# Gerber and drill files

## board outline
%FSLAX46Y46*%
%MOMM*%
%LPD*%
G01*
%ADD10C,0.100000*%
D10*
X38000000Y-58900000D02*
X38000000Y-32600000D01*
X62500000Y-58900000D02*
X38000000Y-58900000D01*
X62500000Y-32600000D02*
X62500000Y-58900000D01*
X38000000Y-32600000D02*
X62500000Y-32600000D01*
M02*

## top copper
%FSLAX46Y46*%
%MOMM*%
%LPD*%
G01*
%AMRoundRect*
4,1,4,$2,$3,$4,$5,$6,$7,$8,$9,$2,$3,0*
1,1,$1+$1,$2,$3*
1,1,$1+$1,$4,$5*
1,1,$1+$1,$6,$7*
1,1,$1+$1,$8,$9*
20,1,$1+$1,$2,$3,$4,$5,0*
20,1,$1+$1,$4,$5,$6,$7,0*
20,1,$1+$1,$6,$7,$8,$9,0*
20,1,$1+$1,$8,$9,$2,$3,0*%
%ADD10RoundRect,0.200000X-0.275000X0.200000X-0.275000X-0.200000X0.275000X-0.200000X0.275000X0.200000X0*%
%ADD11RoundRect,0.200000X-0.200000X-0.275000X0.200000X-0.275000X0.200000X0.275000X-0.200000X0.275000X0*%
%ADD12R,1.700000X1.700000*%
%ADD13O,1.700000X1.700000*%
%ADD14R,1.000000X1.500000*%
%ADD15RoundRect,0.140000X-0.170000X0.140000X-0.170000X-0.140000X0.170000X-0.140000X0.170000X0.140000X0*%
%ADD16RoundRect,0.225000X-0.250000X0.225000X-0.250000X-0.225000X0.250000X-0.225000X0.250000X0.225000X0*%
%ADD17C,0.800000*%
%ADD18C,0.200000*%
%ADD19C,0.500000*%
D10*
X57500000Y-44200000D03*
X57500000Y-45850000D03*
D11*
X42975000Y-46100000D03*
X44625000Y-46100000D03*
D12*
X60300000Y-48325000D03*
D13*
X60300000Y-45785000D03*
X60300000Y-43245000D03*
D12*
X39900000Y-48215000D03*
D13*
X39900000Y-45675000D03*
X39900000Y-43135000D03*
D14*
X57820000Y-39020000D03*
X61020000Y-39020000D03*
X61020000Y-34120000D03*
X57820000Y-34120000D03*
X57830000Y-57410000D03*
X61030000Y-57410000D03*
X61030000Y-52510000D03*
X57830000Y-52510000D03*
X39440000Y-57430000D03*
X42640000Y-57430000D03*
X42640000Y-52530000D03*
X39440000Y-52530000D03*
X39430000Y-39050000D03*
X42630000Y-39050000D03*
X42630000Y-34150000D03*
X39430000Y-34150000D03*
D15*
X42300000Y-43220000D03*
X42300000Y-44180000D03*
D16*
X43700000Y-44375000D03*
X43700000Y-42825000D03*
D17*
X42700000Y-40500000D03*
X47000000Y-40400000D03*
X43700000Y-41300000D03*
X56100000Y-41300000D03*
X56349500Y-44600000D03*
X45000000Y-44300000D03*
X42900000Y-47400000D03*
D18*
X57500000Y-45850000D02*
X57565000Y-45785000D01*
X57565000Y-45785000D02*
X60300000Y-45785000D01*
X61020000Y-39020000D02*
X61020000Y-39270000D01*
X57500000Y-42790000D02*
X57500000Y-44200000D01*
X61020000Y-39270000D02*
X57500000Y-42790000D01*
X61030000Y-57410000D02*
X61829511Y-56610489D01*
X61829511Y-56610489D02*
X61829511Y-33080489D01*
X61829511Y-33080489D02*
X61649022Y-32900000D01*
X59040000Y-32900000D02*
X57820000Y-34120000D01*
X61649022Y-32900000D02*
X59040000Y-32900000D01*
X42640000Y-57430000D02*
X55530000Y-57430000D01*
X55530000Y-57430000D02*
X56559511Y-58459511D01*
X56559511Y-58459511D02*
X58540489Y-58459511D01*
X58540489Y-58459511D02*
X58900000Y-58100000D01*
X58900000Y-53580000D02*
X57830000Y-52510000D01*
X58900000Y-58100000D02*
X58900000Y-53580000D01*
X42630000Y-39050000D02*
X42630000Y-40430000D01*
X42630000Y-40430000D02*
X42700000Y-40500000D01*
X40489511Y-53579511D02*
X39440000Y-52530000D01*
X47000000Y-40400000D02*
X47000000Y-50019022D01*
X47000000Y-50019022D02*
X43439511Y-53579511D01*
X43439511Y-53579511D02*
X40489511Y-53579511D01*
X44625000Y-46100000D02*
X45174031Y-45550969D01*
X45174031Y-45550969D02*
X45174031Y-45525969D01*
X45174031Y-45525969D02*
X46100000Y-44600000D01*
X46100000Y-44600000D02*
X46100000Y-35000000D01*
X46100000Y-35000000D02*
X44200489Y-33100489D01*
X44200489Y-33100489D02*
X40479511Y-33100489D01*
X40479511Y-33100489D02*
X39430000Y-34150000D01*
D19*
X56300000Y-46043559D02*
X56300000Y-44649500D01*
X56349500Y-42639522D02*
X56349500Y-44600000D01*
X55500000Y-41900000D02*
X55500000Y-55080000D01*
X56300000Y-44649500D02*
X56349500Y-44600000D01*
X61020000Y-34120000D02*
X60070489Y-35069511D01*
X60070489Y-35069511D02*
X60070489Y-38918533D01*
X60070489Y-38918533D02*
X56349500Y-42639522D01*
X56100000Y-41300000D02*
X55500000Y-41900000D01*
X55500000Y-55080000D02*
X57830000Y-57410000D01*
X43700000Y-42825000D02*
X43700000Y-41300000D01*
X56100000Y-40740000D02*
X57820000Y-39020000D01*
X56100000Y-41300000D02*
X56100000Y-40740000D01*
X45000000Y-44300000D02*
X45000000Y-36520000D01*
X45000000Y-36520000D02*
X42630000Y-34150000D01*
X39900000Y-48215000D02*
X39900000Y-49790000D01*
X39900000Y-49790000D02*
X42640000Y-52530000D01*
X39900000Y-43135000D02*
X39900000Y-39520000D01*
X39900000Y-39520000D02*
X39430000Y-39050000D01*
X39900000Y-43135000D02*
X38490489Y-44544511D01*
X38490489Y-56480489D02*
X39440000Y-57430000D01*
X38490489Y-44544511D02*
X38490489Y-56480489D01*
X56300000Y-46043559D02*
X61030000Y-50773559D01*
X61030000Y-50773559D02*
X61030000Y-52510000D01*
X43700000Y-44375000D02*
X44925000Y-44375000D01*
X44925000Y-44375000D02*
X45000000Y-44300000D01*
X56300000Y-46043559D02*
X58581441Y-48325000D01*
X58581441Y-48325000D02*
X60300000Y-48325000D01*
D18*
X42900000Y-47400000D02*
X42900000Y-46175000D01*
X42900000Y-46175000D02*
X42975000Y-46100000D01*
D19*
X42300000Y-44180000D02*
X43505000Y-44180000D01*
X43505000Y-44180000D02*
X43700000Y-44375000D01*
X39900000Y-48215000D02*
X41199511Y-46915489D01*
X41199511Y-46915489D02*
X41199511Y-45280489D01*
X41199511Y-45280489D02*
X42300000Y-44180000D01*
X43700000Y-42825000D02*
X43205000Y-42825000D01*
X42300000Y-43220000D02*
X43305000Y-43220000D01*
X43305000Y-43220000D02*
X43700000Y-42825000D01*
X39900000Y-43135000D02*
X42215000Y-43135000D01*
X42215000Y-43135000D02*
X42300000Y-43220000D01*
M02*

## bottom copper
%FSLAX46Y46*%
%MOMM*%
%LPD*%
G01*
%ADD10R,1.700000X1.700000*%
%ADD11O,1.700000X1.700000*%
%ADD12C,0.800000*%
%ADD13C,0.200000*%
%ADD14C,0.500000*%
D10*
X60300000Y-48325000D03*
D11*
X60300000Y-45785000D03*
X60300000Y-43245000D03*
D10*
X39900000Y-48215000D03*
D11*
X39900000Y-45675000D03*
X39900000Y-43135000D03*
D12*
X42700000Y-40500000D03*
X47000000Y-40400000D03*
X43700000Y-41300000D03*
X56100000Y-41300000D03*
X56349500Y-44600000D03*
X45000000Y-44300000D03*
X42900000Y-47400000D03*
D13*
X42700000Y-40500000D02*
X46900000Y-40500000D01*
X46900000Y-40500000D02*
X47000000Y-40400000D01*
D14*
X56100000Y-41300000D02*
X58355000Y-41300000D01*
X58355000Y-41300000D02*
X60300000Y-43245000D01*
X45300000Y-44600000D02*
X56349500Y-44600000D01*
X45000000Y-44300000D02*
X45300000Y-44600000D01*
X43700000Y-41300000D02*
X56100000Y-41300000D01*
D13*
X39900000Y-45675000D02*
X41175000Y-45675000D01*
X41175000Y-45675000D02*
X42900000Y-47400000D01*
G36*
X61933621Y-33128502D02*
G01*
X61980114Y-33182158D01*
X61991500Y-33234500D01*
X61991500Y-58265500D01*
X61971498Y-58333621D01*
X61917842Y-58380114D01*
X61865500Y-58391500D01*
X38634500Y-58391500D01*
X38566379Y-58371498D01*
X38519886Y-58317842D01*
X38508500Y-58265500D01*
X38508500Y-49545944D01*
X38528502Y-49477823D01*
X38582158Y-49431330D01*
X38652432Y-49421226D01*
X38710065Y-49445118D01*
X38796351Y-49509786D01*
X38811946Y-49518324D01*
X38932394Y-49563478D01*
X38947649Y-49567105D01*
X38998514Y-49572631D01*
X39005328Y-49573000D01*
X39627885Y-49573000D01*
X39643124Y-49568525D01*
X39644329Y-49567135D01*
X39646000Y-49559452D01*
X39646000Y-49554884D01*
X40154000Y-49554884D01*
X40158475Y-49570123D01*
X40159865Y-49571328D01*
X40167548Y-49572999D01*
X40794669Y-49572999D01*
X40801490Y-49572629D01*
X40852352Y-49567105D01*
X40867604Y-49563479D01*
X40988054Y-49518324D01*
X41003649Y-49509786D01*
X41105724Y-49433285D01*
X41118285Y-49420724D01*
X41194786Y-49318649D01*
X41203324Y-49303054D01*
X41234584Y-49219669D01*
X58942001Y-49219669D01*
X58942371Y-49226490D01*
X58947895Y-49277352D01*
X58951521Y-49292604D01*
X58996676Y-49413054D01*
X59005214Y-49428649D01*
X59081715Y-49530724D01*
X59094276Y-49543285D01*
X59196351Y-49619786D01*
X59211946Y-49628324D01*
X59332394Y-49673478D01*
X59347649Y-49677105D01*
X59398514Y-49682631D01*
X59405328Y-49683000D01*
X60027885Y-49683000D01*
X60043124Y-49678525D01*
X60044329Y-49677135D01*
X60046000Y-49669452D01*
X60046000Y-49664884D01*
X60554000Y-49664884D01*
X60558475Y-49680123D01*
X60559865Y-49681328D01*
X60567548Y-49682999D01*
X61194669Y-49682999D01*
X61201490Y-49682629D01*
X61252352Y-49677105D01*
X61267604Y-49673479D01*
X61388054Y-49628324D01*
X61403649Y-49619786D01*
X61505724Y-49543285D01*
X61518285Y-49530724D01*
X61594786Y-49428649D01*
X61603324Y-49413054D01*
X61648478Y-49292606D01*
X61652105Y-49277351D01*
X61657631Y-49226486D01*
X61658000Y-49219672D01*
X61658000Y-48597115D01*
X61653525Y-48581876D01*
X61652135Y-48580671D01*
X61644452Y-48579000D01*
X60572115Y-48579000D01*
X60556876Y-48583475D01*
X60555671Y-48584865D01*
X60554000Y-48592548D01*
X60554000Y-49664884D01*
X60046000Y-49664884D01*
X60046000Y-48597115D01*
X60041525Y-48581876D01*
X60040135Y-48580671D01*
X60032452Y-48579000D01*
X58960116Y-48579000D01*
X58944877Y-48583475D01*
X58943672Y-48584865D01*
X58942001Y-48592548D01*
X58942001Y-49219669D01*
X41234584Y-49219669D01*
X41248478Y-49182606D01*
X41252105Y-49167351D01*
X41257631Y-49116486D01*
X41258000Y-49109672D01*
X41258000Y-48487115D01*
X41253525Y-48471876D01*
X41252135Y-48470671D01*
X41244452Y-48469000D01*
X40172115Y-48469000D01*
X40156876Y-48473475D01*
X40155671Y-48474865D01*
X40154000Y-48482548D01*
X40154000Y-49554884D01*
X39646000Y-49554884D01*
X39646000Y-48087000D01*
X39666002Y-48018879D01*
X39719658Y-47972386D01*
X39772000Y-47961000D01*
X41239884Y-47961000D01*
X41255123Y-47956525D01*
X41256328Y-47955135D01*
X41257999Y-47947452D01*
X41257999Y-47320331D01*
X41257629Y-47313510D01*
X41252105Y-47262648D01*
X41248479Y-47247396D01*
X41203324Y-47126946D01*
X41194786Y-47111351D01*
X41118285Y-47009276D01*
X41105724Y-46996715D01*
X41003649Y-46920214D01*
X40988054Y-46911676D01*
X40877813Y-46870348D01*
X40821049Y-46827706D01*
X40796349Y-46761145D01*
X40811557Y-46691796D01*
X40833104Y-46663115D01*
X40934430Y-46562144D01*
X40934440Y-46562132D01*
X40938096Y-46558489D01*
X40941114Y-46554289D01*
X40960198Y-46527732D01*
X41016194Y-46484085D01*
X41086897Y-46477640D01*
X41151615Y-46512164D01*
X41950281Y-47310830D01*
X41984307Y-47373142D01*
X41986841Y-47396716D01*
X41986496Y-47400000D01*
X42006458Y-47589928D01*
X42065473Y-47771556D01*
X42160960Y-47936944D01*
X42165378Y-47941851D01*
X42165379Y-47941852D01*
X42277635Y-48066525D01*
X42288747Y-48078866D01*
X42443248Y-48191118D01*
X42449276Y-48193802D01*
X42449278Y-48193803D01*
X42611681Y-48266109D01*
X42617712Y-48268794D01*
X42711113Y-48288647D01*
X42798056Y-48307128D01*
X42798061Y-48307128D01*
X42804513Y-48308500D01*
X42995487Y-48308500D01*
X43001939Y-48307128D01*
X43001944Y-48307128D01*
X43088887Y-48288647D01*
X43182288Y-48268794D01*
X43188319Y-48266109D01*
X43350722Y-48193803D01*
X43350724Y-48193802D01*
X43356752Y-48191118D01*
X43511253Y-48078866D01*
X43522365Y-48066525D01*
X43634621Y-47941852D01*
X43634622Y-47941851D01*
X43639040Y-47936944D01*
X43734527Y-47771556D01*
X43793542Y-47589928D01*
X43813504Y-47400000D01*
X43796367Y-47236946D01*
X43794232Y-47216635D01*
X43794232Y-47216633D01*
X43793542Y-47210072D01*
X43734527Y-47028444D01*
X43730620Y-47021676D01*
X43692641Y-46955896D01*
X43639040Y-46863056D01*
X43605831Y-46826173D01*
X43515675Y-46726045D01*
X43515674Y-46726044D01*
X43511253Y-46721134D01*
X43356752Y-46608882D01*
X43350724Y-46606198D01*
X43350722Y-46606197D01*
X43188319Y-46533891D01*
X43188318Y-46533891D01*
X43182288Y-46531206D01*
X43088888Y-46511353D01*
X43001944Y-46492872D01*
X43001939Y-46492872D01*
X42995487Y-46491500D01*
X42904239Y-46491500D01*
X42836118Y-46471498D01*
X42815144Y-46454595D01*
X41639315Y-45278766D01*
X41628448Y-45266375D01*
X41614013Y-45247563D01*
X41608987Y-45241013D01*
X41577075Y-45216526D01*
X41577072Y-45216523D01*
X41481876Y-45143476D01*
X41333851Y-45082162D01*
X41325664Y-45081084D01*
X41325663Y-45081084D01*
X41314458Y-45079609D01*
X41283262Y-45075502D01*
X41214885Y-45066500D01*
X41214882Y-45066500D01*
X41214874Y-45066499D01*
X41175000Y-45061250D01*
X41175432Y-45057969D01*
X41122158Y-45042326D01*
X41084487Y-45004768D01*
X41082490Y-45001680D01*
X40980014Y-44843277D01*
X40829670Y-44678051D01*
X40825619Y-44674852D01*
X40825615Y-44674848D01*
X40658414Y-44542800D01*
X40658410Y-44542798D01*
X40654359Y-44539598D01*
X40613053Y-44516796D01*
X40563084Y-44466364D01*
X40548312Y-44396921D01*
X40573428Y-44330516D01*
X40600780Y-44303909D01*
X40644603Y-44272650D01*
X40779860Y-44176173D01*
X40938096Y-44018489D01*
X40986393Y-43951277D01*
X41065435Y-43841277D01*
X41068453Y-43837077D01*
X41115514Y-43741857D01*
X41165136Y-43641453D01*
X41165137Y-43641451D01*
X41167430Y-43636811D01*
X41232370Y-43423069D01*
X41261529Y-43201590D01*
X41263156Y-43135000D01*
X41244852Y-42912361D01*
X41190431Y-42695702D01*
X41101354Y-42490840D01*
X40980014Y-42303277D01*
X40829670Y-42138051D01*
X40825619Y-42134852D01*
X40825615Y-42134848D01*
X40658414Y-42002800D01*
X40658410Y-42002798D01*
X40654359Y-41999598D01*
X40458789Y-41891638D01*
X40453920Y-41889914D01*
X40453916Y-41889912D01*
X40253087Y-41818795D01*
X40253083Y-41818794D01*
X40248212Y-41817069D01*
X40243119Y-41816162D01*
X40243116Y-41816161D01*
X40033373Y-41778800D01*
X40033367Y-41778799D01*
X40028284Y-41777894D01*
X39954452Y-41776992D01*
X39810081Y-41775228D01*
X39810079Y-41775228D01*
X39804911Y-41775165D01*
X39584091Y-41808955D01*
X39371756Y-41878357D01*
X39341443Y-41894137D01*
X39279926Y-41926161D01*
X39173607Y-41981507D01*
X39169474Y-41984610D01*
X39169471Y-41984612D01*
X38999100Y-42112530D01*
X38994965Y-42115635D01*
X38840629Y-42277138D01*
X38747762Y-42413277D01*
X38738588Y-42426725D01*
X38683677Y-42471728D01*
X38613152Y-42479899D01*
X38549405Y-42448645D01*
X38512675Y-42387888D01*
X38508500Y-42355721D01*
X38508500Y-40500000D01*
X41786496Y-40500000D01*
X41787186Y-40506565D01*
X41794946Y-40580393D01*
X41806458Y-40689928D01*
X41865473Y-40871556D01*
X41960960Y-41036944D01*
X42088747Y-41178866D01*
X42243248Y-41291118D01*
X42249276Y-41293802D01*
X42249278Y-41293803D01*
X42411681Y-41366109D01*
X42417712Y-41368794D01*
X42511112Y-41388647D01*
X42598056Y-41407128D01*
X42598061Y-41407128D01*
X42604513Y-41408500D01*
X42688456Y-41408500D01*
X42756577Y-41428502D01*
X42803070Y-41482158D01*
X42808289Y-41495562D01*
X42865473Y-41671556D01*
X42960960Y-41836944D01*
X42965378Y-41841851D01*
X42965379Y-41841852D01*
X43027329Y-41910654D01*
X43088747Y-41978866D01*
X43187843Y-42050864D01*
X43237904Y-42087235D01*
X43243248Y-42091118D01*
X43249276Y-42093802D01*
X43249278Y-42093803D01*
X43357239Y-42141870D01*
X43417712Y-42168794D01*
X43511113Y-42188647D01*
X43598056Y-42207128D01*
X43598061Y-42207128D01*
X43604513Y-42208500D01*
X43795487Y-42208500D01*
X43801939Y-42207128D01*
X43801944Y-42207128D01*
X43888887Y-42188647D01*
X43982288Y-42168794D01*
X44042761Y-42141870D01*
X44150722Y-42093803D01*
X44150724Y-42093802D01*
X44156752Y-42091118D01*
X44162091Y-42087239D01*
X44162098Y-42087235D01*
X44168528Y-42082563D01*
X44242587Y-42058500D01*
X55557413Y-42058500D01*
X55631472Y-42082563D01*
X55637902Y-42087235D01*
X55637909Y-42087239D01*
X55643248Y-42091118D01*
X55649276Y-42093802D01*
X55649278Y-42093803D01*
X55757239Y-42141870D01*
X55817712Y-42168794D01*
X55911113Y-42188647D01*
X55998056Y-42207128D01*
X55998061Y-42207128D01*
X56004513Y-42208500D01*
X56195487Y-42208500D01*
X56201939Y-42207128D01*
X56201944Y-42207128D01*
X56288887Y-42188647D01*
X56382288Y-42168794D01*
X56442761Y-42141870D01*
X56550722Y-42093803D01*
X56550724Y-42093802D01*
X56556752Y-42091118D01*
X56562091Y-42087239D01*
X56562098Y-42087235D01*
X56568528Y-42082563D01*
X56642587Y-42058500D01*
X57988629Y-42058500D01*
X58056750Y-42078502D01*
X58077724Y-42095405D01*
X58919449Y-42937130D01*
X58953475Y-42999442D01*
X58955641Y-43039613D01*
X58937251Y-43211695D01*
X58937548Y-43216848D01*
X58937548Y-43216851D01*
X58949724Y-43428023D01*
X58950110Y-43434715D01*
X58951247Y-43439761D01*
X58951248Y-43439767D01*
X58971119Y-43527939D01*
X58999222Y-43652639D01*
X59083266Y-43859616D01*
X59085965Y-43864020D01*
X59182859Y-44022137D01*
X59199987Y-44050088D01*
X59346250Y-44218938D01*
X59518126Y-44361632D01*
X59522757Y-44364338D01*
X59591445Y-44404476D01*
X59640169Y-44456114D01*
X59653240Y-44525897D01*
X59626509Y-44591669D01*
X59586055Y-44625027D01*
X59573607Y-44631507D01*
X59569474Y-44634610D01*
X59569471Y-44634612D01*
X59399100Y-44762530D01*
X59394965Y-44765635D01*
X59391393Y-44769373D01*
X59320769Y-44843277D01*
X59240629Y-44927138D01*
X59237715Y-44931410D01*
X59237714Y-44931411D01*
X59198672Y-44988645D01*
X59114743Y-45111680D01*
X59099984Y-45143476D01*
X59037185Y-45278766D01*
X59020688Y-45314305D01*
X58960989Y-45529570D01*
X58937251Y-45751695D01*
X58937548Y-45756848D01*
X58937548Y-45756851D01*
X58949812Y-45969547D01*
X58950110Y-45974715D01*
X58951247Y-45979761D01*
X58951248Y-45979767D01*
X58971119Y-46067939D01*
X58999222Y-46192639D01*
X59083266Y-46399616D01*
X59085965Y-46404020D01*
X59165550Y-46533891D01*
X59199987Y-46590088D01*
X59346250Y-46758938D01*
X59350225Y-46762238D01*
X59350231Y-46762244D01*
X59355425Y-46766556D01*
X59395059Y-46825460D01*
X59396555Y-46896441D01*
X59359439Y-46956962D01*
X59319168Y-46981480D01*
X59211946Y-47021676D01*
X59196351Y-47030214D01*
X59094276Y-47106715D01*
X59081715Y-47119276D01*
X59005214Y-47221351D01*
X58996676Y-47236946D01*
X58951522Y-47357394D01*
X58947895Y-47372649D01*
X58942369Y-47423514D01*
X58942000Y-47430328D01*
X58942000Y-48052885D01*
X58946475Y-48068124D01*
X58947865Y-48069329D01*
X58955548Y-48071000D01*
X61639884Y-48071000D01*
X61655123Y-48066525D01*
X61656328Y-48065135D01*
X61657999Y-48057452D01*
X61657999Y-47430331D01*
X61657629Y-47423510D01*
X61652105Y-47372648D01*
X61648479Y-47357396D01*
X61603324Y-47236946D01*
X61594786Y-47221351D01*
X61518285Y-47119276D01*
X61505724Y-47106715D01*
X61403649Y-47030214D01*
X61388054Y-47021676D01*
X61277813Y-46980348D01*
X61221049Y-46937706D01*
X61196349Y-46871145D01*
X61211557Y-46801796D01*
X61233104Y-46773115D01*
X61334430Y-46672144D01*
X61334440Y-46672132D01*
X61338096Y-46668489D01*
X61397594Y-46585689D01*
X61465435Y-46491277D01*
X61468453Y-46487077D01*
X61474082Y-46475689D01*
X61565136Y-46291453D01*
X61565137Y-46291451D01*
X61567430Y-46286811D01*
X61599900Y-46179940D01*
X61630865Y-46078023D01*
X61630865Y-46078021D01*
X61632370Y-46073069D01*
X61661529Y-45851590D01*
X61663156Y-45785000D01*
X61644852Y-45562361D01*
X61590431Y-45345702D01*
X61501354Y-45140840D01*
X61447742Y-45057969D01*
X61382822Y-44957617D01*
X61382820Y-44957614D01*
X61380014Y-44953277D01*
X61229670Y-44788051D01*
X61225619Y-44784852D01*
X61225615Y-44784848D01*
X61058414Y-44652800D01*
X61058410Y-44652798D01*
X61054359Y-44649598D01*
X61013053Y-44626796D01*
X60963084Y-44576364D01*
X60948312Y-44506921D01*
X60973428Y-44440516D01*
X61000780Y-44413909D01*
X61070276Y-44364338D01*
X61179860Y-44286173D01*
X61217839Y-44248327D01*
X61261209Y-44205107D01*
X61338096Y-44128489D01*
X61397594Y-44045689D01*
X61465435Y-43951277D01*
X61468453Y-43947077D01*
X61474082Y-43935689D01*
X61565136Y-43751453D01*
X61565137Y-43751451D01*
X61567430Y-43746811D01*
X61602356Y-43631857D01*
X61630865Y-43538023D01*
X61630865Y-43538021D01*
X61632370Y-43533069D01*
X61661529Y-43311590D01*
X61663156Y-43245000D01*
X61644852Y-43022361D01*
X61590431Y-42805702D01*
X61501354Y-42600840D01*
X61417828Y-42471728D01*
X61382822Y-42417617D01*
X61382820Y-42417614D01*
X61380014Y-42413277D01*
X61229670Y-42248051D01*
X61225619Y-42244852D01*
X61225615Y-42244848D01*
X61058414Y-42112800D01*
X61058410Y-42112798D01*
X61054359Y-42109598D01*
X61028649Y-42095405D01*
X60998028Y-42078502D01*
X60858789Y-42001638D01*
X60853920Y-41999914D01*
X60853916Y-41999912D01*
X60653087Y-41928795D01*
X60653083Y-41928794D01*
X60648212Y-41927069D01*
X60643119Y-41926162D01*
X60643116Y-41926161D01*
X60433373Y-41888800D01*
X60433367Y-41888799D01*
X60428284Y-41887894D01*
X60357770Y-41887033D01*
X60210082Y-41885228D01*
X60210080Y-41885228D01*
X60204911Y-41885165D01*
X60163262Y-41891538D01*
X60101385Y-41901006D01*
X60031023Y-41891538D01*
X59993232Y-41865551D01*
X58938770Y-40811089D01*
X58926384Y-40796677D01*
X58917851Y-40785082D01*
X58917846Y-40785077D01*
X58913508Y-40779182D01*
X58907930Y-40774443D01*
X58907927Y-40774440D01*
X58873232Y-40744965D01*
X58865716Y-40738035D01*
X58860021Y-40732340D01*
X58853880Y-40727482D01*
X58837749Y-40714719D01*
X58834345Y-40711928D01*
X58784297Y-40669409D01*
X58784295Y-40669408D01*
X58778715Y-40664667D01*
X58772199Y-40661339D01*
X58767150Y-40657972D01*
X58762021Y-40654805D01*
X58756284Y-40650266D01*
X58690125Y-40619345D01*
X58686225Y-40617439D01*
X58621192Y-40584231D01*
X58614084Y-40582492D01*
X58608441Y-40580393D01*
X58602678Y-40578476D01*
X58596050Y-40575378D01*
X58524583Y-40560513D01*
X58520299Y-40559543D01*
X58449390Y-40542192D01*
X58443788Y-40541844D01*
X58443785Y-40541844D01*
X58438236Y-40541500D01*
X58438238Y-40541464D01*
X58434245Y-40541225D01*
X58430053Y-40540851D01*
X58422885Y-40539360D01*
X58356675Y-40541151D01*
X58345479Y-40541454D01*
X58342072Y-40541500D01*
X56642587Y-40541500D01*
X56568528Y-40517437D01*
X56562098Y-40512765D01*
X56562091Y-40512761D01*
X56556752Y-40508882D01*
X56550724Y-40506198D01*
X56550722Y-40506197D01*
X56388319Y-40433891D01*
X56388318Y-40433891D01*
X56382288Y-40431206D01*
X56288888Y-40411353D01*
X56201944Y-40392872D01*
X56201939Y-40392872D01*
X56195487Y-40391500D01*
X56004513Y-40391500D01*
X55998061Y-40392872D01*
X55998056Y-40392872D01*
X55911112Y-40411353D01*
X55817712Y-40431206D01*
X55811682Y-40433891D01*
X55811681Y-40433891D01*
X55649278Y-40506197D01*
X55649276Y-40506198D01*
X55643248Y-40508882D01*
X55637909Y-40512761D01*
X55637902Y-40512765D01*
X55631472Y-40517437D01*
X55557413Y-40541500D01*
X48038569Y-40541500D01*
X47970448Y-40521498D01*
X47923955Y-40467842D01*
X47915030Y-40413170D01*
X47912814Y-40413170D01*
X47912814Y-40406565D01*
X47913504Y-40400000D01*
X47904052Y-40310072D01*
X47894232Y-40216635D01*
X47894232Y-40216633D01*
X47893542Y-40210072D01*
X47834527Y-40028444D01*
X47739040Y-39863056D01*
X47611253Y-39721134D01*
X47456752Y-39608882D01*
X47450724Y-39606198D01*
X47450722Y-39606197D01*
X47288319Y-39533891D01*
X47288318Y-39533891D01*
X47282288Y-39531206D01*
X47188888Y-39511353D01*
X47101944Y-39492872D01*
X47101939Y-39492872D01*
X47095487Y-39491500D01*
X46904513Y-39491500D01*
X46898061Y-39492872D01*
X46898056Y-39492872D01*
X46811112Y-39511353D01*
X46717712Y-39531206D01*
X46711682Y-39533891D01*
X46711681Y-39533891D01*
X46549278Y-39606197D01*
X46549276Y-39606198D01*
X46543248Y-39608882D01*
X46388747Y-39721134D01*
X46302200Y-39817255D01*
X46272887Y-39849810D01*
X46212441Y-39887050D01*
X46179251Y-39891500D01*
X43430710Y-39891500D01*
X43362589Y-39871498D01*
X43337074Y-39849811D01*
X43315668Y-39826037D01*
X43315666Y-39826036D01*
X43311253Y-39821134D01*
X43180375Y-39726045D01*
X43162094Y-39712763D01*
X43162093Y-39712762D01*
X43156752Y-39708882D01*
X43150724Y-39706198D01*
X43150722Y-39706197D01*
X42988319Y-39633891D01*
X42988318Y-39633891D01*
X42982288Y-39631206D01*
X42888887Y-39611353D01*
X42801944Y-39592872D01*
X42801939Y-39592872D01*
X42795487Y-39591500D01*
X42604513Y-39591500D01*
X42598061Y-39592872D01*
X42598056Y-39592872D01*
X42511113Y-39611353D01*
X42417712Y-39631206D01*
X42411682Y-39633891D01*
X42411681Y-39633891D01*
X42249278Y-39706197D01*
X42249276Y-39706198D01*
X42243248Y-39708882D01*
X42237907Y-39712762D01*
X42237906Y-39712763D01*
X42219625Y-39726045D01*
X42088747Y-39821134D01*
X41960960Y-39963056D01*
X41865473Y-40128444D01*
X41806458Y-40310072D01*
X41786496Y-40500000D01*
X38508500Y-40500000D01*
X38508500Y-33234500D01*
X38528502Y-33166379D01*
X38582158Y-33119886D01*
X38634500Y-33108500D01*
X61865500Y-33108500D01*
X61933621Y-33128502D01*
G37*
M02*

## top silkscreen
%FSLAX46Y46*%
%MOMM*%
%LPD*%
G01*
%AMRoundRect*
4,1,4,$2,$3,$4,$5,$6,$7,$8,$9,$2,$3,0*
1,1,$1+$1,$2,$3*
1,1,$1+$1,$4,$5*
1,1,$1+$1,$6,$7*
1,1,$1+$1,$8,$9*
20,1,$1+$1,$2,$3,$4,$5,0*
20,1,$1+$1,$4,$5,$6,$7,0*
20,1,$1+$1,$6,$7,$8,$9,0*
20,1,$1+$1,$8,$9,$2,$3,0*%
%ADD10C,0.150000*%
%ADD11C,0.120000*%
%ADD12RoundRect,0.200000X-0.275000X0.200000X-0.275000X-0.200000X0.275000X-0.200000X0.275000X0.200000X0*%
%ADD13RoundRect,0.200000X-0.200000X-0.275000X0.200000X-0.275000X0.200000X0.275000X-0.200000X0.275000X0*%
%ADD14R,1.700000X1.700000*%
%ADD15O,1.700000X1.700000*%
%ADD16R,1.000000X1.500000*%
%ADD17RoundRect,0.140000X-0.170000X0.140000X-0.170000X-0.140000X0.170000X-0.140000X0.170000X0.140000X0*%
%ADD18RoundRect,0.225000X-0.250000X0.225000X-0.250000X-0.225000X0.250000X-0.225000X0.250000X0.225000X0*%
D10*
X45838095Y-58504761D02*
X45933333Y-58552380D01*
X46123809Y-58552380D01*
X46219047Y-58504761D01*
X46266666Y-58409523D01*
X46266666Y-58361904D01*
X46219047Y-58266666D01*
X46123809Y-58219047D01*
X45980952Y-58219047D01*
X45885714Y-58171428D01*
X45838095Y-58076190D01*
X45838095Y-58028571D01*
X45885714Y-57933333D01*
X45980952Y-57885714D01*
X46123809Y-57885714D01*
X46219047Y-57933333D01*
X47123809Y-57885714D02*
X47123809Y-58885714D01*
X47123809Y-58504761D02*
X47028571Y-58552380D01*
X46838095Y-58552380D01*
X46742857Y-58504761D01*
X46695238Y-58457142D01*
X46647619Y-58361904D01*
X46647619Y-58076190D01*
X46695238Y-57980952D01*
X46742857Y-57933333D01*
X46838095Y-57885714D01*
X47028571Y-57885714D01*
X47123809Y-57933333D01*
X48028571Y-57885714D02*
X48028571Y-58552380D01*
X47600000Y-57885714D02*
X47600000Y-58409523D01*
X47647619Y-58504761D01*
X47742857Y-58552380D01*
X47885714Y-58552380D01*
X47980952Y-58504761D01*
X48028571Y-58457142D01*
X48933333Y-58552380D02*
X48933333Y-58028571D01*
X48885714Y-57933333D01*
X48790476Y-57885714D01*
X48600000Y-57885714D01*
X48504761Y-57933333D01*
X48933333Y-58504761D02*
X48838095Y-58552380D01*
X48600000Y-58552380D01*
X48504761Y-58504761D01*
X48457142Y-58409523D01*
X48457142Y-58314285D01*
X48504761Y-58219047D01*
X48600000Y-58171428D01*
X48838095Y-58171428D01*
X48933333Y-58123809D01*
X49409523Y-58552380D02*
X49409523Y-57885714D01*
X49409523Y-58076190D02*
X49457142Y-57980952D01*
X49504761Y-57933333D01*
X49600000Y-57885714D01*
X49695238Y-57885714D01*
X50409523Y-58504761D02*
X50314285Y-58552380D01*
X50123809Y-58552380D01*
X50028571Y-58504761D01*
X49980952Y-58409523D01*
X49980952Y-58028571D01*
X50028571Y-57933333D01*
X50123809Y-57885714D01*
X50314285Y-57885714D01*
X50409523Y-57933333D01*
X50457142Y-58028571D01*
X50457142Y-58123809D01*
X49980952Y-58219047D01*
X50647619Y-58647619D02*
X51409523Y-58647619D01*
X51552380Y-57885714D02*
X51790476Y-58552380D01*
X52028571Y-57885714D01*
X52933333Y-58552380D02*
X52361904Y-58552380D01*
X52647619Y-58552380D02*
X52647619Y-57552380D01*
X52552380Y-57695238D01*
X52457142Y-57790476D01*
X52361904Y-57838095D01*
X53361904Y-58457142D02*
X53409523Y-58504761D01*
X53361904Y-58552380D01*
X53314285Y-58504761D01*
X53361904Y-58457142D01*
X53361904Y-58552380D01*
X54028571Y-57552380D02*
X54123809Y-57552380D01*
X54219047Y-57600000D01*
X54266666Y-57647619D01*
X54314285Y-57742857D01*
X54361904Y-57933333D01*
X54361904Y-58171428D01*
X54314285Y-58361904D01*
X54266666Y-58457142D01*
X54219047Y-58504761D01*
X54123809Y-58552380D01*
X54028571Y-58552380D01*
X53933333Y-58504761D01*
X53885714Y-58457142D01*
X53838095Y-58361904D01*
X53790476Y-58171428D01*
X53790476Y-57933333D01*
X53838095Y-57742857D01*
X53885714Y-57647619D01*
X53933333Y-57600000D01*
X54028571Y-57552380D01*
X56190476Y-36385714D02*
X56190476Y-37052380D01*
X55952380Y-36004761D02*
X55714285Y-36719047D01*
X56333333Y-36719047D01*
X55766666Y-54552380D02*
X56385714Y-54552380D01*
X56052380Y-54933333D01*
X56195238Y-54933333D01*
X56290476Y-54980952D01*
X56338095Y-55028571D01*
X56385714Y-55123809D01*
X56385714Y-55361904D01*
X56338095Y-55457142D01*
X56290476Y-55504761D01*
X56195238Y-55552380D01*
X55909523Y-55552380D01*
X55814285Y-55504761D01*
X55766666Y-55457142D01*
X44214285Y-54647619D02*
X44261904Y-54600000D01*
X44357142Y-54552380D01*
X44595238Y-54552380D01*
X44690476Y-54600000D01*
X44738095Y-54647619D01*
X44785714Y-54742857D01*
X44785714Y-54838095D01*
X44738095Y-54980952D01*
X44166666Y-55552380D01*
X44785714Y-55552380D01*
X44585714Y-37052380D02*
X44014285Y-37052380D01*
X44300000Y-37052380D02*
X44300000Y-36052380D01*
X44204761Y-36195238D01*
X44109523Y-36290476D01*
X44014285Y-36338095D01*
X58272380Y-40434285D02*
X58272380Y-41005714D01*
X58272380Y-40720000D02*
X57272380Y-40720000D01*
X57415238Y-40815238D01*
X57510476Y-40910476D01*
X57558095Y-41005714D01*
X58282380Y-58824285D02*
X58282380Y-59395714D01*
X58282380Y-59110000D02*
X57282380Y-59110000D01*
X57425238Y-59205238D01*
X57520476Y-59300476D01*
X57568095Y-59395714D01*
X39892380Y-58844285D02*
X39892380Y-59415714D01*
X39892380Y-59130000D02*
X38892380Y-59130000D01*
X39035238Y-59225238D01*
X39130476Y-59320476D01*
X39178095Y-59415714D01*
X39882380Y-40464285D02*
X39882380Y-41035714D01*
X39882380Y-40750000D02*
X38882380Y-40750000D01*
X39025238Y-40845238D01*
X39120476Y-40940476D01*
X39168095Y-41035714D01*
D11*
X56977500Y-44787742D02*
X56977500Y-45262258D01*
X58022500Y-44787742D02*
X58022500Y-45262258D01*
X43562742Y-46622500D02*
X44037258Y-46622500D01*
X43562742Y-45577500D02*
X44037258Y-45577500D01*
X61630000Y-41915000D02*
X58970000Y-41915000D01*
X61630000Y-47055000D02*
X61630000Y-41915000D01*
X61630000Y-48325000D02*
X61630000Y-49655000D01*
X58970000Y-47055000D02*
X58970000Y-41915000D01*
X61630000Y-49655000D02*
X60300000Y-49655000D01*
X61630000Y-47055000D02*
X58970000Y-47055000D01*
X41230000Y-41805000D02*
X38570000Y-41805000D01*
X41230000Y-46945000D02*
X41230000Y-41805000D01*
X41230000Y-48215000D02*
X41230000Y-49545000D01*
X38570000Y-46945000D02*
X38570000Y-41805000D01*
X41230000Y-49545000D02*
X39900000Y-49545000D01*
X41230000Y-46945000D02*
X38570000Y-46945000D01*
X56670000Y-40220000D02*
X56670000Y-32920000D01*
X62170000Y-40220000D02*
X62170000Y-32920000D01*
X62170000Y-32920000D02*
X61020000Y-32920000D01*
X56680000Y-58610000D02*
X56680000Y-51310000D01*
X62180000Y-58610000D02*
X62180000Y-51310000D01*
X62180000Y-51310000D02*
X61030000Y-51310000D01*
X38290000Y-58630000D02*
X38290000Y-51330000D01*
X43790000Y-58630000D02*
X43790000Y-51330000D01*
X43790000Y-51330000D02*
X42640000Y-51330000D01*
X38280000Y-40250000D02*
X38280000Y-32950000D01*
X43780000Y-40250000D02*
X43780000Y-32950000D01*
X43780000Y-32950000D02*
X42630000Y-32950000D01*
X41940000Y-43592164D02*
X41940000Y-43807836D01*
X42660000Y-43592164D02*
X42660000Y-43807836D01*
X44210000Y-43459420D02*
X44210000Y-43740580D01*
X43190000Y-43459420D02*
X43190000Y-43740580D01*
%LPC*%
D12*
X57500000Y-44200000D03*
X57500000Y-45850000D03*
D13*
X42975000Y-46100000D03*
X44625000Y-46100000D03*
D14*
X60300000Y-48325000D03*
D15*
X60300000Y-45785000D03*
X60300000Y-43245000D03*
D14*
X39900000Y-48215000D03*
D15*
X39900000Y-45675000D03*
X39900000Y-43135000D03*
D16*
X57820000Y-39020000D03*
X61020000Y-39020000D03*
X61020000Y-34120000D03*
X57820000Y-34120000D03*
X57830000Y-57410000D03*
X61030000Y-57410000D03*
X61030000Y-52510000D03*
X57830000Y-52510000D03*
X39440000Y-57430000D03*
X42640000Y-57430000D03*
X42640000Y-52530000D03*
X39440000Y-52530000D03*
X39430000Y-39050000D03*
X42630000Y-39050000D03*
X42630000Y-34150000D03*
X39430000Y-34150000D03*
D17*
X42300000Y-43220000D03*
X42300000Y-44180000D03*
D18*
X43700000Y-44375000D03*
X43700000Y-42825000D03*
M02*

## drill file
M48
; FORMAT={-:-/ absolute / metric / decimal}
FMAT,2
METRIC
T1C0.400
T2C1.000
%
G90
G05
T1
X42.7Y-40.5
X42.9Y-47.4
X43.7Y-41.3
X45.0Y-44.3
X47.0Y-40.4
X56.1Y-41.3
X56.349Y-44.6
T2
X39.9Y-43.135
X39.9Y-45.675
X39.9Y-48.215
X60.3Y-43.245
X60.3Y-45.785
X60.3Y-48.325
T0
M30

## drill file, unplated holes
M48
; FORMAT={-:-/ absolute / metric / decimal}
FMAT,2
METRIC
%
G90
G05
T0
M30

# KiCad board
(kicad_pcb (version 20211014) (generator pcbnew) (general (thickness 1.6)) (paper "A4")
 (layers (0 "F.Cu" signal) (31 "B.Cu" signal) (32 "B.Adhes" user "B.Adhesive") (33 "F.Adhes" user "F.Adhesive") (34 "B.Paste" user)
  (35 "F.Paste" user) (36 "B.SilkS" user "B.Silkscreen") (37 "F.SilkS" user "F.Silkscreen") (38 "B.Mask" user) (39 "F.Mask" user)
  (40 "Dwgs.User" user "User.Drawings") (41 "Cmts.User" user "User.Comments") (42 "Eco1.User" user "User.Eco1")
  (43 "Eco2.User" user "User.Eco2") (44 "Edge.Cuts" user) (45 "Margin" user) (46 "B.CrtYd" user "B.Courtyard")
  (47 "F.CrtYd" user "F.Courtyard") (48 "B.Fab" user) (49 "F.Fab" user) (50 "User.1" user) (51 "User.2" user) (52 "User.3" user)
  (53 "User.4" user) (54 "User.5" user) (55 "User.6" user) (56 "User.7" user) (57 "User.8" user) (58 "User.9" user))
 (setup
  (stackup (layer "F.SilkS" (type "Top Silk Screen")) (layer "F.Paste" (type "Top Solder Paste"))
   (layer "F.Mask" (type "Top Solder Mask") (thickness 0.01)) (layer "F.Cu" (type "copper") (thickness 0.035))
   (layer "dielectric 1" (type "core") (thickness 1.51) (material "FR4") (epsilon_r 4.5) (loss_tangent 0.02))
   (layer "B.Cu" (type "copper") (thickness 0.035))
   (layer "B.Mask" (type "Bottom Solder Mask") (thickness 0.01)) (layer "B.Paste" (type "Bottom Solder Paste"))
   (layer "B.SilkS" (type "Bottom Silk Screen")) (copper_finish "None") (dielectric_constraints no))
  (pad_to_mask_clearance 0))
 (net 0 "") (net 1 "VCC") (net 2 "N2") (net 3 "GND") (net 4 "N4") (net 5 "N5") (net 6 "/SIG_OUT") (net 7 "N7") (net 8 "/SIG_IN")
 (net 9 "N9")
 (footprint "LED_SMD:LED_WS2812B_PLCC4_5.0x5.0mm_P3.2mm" (layer "F.Cu") (at 41.03 36.6 90)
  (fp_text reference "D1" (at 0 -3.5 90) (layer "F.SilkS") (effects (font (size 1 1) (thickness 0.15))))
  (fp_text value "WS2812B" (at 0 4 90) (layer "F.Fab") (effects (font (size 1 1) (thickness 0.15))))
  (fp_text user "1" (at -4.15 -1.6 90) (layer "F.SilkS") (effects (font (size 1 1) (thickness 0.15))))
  (fp_line (start -3.65 -2.75) (end 3.65 -2.75) (layer "F.SilkS") (width 0.12))
  (fp_line (start 3.65 2.75) (end 3.65 1.6) (layer "F.SilkS") (width 0.12))
  (fp_line (start -3.65 2.75) (end 3.65 2.75) (layer "F.SilkS") (width 0.12))
  (pad "1" smd rect (at -2.45 -1.6 90) (size 1.5 1) (layers "F.Cu" "F.Paste" "F.Mask") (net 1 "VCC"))
  (pad "2" smd rect (at -2.45 1.6 90) (size 1.5 1) (layers "F.Cu" "F.Paste" "F.Mask") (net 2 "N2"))
  (pad "3" smd rect (at 2.45 1.6 90) (size 1.5 1) (layers "F.Cu" "F.Paste" "F.Mask") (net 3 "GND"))
  (pad "4" smd rect (at 2.45 -1.6 90) (size 1.5 1) (layers "F.Cu" "F.Paste" "F.Mask") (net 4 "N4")))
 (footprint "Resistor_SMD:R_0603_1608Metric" (layer "F.Cu") (at 57.5 45.025 -90)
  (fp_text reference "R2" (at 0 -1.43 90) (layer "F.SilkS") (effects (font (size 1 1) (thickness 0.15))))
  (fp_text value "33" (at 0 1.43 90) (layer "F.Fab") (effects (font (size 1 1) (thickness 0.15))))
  (fp_line (start -0.237258 -0.5225) (end 0.237258 -0.5225) (layer "F.SilkS") (width 0.12))
  (fp_line (start -0.237258 0.5225) (end 0.237258 0.5225) (layer "F.SilkS") (width 0.12))
  (pad "1" smd roundrect (at -0.825 0 270) (size 0.8 0.95) (layers "F.Cu" "F.Paste" "F.Mask") (roundrect_rratio 0.25) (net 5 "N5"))
  (pad "2" smd roundrect (at 0.825 0 270) (size 0.8 0.95) (layers "F.Cu" "F.Paste" "F.Mask") (roundrect_rratio 0.25) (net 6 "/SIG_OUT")))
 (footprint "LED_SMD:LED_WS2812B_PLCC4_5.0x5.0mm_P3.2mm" (layer "F.Cu") (at 41.04 54.98 90)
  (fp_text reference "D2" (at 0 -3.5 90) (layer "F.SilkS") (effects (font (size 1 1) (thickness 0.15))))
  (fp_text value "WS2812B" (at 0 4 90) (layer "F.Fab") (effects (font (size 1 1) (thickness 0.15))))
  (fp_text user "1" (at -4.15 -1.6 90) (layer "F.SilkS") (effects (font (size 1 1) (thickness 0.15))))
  (fp_line (start 3.65 2.75) (end 3.65 1.6) (layer "F.SilkS") (width 0.12))
  (fp_line (start -3.65 2.75) (end 3.65 2.75) (layer "F.SilkS") (width 0.12))
  (fp_line (start -3.65 -2.75) (end 3.65 -2.75) (layer "F.SilkS") (width 0.12))
  (pad "1" smd rect (at -2.45 -1.6 90) (size 1.5 1) (layers "F.Cu" "F.Paste" "F.Mask") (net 1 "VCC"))
  (pad "2" smd rect (at -2.45 1.6 90) (size 1.5 1) (layers "F.Cu" "F.Paste" "F.Mask") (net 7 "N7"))
  (pad "3" smd rect (at 2.45 1.6 90) (size 1.5 1) (layers "F.Cu" "F.Paste" "F.Mask") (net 3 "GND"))
  (pad "4" smd rect (at 2.45 -1.6 90) (size 1.5 1) (layers "F.Cu" "F.Paste" "F.Mask") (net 2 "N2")))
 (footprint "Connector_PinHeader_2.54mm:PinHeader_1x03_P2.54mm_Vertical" (layer "F.Cu") (at 60.3 48.325 180)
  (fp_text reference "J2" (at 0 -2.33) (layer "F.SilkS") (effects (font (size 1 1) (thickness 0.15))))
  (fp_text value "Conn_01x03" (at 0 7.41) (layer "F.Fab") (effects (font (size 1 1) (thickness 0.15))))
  (fp_line (start -1.33 1.27) (end 1.33 1.27) (layer "F.SilkS") (width 0.12))
  (fp_line (start -1.33 1.27) (end -1.33 6.41) (layer "F.SilkS") (width 0.12))
  (fp_line (start -1.33 0) (end -1.33 -1.33) (layer "F.SilkS") (width 0.12))
  (fp_line (start -1.33 -1.33) (end 0 -1.33) (layer "F.SilkS") (width 0.12))
  (fp_line (start -1.33 6.41) (end 1.33 6.41) (layer "F.SilkS") (width 0.12))
  (fp_line (start 1.33 1.27) (end 1.33 6.41) (layer "F.SilkS") (width 0.12))
  (pad "1" thru_hole rect (at 0 0 180) (size 1.7 1.7) (drill 1) (layers *.Cu *.Mask) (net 3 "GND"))
  (pad "2" thru_hole oval (at 0 2.54 180) (size 1.7 1.7) (drill 1) (layers *.Cu *.Mask) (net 6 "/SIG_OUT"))
  (pad "3" thru_hole oval (at 0 5.08 180) (size 1.7 1.7) (drill 1) (layers *.Cu *.Mask) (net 1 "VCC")))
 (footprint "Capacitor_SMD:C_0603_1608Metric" (layer "F.Cu") (at 43.7 43.6 -90)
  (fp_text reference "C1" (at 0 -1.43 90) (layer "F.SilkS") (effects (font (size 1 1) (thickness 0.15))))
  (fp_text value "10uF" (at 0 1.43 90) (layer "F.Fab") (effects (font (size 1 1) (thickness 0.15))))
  (fp_line (start -0.14058 0.51) (end 0.14058 0.51) (layer "F.SilkS") (width 0.12))
  (fp_line (start -0.14058 -0.51) (end 0.14058 -0.51) (layer "F.SilkS") (width 0.12))
  (pad "1" smd roundrect (at -0.775 0 270) (size 0.9 0.95) (layers "F.Cu" "F.Paste" "F.Mask") (roundrect_rratio 0.25) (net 1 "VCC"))
  (pad "2" smd roundrect (at 0.775 0 270) (size 0.9 0.95) (layers "F.Cu" "F.Paste" "F.Mask") (roundrect_rratio 0.25) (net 3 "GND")))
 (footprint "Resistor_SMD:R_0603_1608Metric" (layer "F.Cu") (at 43.8 46.1)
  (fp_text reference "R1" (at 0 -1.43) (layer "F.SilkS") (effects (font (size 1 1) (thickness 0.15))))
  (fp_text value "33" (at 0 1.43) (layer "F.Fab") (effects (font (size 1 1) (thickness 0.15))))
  (fp_line (start -0.237258 -0.5225) (end 0.237258 -0.5225) (layer "F.SilkS") (width 0.12))
  (fp_line (start -0.237258 0.5225) (end 0.237258 0.5225) (layer "F.SilkS") (width 0.12))
  (pad "1" smd roundrect (at -0.825 0) (size 0.8 0.95) (layers "F.Cu" "F.Paste" "F.Mask") (roundrect_rratio 0.25) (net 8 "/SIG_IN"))
  (pad "2" smd roundrect (at 0.825 0) (size 0.8 0.95) (layers "F.Cu" "F.Paste" "F.Mask") (roundrect_rratio 0.25) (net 4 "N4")))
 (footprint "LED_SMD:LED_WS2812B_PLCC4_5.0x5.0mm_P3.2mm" (layer "F.Cu") (at 59.43 54.96 90)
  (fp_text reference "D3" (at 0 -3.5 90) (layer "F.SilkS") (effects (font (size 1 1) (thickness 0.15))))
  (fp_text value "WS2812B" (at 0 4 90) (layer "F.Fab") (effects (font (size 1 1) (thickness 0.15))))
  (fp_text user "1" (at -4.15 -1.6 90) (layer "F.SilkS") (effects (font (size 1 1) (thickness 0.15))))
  (fp_line (start 3.65 2.75) (end 3.65 1.6) (layer "F.SilkS") (width 0.12))
  (fp_line (start -3.65 -2.75) (end 3.65 -2.75) (layer "F.SilkS") (width 0.12))
  (fp_line (start -3.65 2.75) (end 3.65 2.75) (layer "F.SilkS") (width 0.12))
  (pad "1" smd rect (at -2.45 -1.6 90) (size 1.5 1) (layers "F.Cu" "F.Paste" "F.Mask") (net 1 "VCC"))
  (pad "2" smd rect (at -2.45 1.6 90) (size 1.5 1) (layers "F.Cu" "F.Paste" "F.Mask") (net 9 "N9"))
  (pad "3" smd rect (at 2.45 1.6 90) (size 1.5 1) (layers "F.Cu" "F.Paste" "F.Mask") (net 3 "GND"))
  (pad "4" smd rect (at 2.45 -1.6 90) (size 1.5 1) (layers "F.Cu" "F.Paste" "F.Mask") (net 7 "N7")))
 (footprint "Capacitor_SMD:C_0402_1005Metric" (layer "F.Cu") (at 42.3 43.7 -90)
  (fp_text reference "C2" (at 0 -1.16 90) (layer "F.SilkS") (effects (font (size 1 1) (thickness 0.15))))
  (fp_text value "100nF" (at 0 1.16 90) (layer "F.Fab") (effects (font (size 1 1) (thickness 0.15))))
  (fp_line (start -0.107836 0.36) (end 0.107836 0.36) (layer "F.SilkS") (width 0.12))
  (fp_line (start -0.107836 -0.36) (end 0.107836 -0.36) (layer "F.SilkS") (width 0.12))
  (pad "1" smd roundrect (at -0.48 0 270) (size 0.56 0.62) (layers "F.Cu" "F.Paste" "F.Mask") (roundrect_rratio 0.25) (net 1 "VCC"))
  (pad "2" smd roundrect (at 0.48 0 270) (size 0.56 0.62) (layers "F.Cu" "F.Paste" "F.Mask") (roundrect_rratio 0.25) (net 3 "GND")))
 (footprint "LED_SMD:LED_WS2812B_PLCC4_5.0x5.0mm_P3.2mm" (layer "F.Cu") (at 59.42 36.57 90)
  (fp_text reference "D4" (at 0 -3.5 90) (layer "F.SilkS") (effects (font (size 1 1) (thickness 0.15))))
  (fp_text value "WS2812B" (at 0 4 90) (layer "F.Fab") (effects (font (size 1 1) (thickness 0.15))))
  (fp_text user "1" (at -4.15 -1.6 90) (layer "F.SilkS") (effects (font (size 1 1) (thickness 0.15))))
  (fp_line (start -3.65 2.75) (end 3.65 2.75) (layer "F.SilkS") (width 0.12))
  (fp_line (start -3.65 -2.75) (end 3.65 -2.75) (layer "F.SilkS") (width 0.12))
  (fp_line (start 3.65 2.75) (end 3.65 1.6) (layer "F.SilkS") (width 0.12))
  (pad "1" smd rect (at -2.45 -1.6 90) (size 1.5 1) (layers "F.Cu" "F.Paste" "F.Mask") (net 1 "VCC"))
  (pad "2" smd rect (at -2.45 1.6 90) (size 1.5 1) (layers "F.Cu" "F.Paste" "F.Mask") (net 5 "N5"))
  (pad "3" smd rect (at 2.45 1.6 90) (size 1.5 1) (layers "F.Cu" "F.Paste" "F.Mask") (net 3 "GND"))
  (pad "4" smd rect (at 2.45 -1.6 90) (size 1.5 1) (layers "F.Cu" "F.Paste" "F.Mask") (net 9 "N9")))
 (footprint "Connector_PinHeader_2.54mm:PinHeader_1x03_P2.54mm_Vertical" (layer "F.Cu") (at 39.9 48.215 180)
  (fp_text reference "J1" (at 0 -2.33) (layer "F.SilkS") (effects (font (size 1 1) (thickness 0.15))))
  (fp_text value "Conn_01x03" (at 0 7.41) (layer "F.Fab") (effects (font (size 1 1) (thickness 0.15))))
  (fp_line (start -1.33 1.27) (end -1.33 6.41) (layer "F.SilkS") (width 0.12))
  (fp_line (start -1.33 0) (end -1.33 -1.33) (layer "F.SilkS") (width 0.12))
  (fp_line (start 1.33 1.27) (end 1.33 6.41) (layer "F.SilkS") (width 0.12))
  (fp_line (start -1.33 6.41) (end 1.33 6.41) (layer "F.SilkS") (width 0.12))
  (fp_line (start -1.33 1.27) (end 1.33 1.27) (layer "F.SilkS") (width 0.12))
  (fp_line (start -1.33 -1.33) (end 0 -1.33) (layer "F.SilkS") (width 0.12))
  (pad "1" thru_hole rect (at 0 0 180) (size 1.7 1.7) (drill 1) (layers *.Cu *.Mask) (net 3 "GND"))
  (pad "2" thru_hole oval (at 0 2.54 180) (size 1.7 1.7) (drill 1) (layers *.Cu *.Mask) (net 8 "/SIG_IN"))
  (pad "3" thru_hole oval (at 0 5.08 180) (size 1.7 1.7) (drill 1) (layers *.Cu *.Mask) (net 1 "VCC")))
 (gr_line (start 38 58.9) (end 38 32.6) (layer "Edge.Cuts") (width 0.1))
 (gr_line (start 62.5 58.9) (end 38 58.9) (layer "Edge.Cuts") (width 0.1))
 (gr_line (start 38 32.6) (end 62.5 32.6) (layer "Edge.Cuts") (width 0.1))
 (gr_line (start 62.5 32.6) (end 62.5 58.9) (layer "Edge.Cuts") (width 0.1))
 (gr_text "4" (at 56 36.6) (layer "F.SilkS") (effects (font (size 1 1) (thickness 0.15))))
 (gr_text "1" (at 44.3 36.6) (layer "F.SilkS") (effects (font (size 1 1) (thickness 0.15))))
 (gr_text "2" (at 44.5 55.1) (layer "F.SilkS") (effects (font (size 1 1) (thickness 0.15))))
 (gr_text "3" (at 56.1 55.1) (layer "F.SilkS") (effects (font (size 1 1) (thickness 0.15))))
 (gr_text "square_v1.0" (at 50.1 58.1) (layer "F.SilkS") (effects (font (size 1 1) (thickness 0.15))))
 (segment (start 39.9 43.135) (end 42.215 43.135) (width 0.5) (layer "F.Cu") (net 1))
 (segment (start 56.1 40.74) (end 57.82 39.02) (width 0.5) (layer "F.Cu") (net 1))
 (segment (start 56.1 41.3) (end 56.1 40.74) (width 0.5) (layer "F.Cu") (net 1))
 (segment (start 43.7 42.825) (end 43.7 41.3) (width 0.5) (layer "F.Cu") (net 1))
 (segment (start 55.5 55.08) (end 57.83 57.41) (width 0.5) (layer "F.Cu") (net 1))
 (segment (start 42.215 43.135) (end 42.3 43.22) (width 0.5) (layer "F.Cu") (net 1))
 (segment (start 39.9 43.135) (end 39.9 39.52) (width 0.5) (layer "F.Cu") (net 1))
 (segment (start 42.3 43.22) (end 43.305 43.22) (width 0.5) (layer "F.Cu") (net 1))
 (segment (start 56.1 41.3) (end 55.5 41.9) (width 0.5) (layer "F.Cu") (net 1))
 (segment (start 38.490489 56.480489) (end 39.44 57.43) (width 0.5) (layer "F.Cu") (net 1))
 (segment (start 43.305 43.22) (end 43.7 42.825) (width 0.5) (layer "F.Cu") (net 1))
 (segment (start 39.9 39.52) (end 39.43 39.05) (width 0.5) (layer "F.Cu") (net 1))
 (segment (start 39.9 43.135) (end 38.490489 44.544511) (width 0.5) (layer "F.Cu") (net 1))
 (segment (start 43.7 42.825) (end 43.205 42.825) (width 0.5) (layer "F.Cu") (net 1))
 (segment (start 38.490489 44.544511) (end 38.490489 56.480489) (width 0.5) (layer "F.Cu") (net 1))
 (segment (start 55.5 41.9) (end 55.5 55.08) (width 0.5) (layer "F.Cu") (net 1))
 (via (at 43.7 41.3) (size 0.8) (drill 0.4) (layers "F.Cu" "B.Cu") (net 1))
 (via (at 56.1 41.3) (size 0.8) (drill 0.4) (layers "F.Cu" "B.Cu") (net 1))
 (segment (start 43.7 41.3) (end 56.1 41.3) (width 0.5) (layer "B.Cu") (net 1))
 (segment (start 58.355 41.3) (end 60.3 43.245) (width 0.5) (layer "B.Cu") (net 1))
 (segment (start 56.1 41.3) (end 58.355 41.3) (width 0.5) (layer "B.Cu") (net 1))
 (segment (start 45 44.3) (end 45 36.52) (width 0.5) (layer "F.Cu") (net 3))
 (segment (start 60.070489 35.069511) (end 60.070489 38.918533) (width 0.5) (layer "F.Cu") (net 3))
 (segment (start 56.3 46.043559) (end 56.3 44.6495) (width 0.5) (layer "F.Cu") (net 3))
 (segment (start 58.581441 48.325) (end 60.3 48.325) (width 0.5) (layer "F.Cu") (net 3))
 (segment (start 56.3 46.043559) (end 58.581441 48.325) (width 0.5) (layer "F.Cu") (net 3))
 (segment (start 43.7 44.375) (end 44.925 44.375) (width 0.5) (layer "F.Cu") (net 3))
 (segment (start 42.3 44.18) (end 43.505 44.18) (width 0.5) (layer "F.Cu") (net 3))
 (segment (start 56.3 44.6495) (end 56.3495 44.6) (width 0.5) (layer "F.Cu") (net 3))
 (segment (start 45 36.52) (end 42.63 34.15) (width 0.5) (layer "F.Cu") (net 3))
 (segment (start 41.199511 45.280489) (end 42.3 44.18) (width 0.5) (layer "F.Cu") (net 3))
 (segment (start 43.505 44.18) (end 43.7 44.375) (width 0.5) (layer "F.Cu") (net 3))
 (segment (start 41.199511 46.915489) (end 41.199511 45.280489) (width 0.5) (layer "F.Cu") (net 3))
 (segment (start 56.3 46.043559) (end 61.03 50.773559) (width 0.5) (layer "F.Cu") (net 3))
 (segment (start 56.3495 42.639522) (end 56.3495 44.6) (width 0.5) (layer "F.Cu") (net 3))
 (segment (start 39.9 48.215) (end 39.9 49.79) (width 0.5) (layer "F.Cu") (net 3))
 (segment (start 61.02 34.12) (end 60.070489 35.069511) (width 0.5) (layer "F.Cu") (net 3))
 (segment (start 39.9 49.79) (end 42.64 52.53) (width 0.5) (layer "F.Cu") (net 3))
 (segment (start 44.925 44.375) (end 45 44.3) (width 0.5) (layer "F.Cu") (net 3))
 (segment (start 60.070489 38.918533) (end 56.3495 42.639522) (width 0.5) (layer "F.Cu") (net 3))
 (segment (start 61.03 50.773559) (end 61.03 52.51) (width 0.5) (layer "F.Cu") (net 3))
 (segment (start 39.9 48.215) (end 41.199511 46.915489) (width 0.5) (layer "F.Cu") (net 3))
 (via (at 45 44.3) (size 0.8) (drill 0.4) (layers "F.Cu" "B.Cu") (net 3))
 (via (at 56.3495 44.6) (size 0.8) (drill 0.4) (layers "F.Cu" "B.Cu") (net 3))
 (segment (start 45 44.3) (end 45.3 44.6) (width 0.5) (layer "B.Cu") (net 3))
 (segment (start 45.3 44.6) (end 56.3495 44.6) (width 0.5) (layer "B.Cu") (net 3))
 (segment (start 42.63 40.43) (end 42.7 40.5) (width 0.2) (layer "F.Cu") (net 2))
 (segment (start 47 50.019022) (end 43.439511 53.579511) (width 0.2) (layer "F.Cu") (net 2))
 (segment (start 42.63 39.05) (end 42.63 40.43) (width 0.2) (layer "F.Cu") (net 2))
 (segment (start 47 40.4) (end 47 50.019022) (width 0.2) (layer "F.Cu") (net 2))
 (segment (start 43.439511 53.579511) (end 40.489511 53.579511) (width 0.2) (layer "F.Cu") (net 2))
 (segment (start 40.489511 53.579511) (end 39.44 52.53) (width 0.2) (layer "F.Cu") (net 2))
 (via (at 42.7 40.5) (size 0.8) (drill 0.4) (layers "F.Cu" "B.Cu") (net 2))
 (via (at 47 40.4) (size 0.8) (drill 0.4) (layers "F.Cu" "B.Cu") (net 2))
 (segment (start 42.7 40.5) (end 46.9 40.5) (width 0.2) (layer "B.Cu") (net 2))
 (segment (start 46.9 40.5) (end 47 40.4) (width 0.2) (layer "B.Cu") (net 2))
 (segment (start 40.479511 33.100489) (end 39.43 34.15) (width 0.2) (layer "F.Cu") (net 4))
 (segment (start 45.174031 45.550969) (end 45.174031 45.525969) (width 0.2) (layer "F.Cu") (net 4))
 (segment (start 46.1 44.6) (end 46.1 35) (width 0.2) (layer "F.Cu") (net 4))
 (segment (start 44.200489 33.100489) (end 40.479511 33.100489) (width 0.2) (layer "F.Cu") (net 4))
 (segment (start 46.1 35) (end 44.200489 33.100489) (width 0.2) (layer "F.Cu") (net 4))
 (segment (start 44.625 46.1) (end 45.174031 45.550969) (width 0.2) (layer "F.Cu") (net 4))
 (segment (start 45.174031 45.525969) (end 46.1 44.6) (width 0.2) (layer "F.Cu") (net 4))
 (segment (start 58.540489 58.459511) (end 58.9 58.1) (width 0.2) (layer "F.Cu") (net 7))
 (segment (start 58.9 53.58) (end 57.83 52.51) (width 0.2) (layer "F.Cu") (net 7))
 (segment (start 56.559511 58.459511) (end 58.540489 58.459511) (width 0.2) (layer "F.Cu") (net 7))
 (segment (start 58.9 58.1) (end 58.9 53.58) (width 0.2) (layer "F.Cu") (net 7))
 (segment (start 42.64 57.43) (end 55.53 57.43) (width 0.2) (layer "F.Cu") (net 7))
 (segment (start 55.53 57.43) (end 56.559511 58.459511) (width 0.2) (layer "F.Cu") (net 7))
 (segment (start 61.03 57.41) (end 61.829511 56.610489) (width 0.2) (layer "F.Cu") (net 9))
 (segment (start 59.04 32.9) (end 57.82 34.12) (width 0.2) (layer "F.Cu") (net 9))
 (segment (start 61.829511 56.610489) (end 61.829511 33.080489) (width 0.2) (layer "F.Cu") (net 9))
 (segment (start 61.829511 33.080489) (end 61.649022 32.9) (width 0.2) (layer "F.Cu") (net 9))
 (segment (start 61.649022 32.9) (end 59.04 32.9) (width 0.2) (layer "F.Cu") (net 9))
 (segment (start 61.02 39.02) (end 61.02 39.27) (width 0.2) (layer "F.Cu") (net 5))
 (segment (start 57.5 42.79) (end 57.5 44.2) (width 0.2) (layer "F.Cu") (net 5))
 (segment (start 61.02 39.27) (end 57.5 42.79) (width 0.2) (layer "F.Cu") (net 5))
 (segment (start 42.9 47.4) (end 42.9 46.175) (width 0.2) (layer "F.Cu") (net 8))
 (segment (start 42.9 46.175) (end 42.975 46.1) (width 0.2) (layer "F.Cu") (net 8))
 (via (at 42.9 47.4) (size 0.8) (drill 0.4) (layers "F.Cu" "B.Cu") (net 8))
 (segment (start 39.9 45.675) (end 41.175 45.675) (width 0.2) (layer "B.Cu") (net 8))
 (segment (start 41.175 45.675) (end 42.9 47.4) (width 0.2) (layer "B.Cu") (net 8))
 (segment (start 57.5 45.85) (end 57.565 45.785) (width 0.2) (layer "F.Cu") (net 6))
 (segment (start 57.565 45.785) (end 60.3 45.785) (width 0.2) (layer "F.Cu") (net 6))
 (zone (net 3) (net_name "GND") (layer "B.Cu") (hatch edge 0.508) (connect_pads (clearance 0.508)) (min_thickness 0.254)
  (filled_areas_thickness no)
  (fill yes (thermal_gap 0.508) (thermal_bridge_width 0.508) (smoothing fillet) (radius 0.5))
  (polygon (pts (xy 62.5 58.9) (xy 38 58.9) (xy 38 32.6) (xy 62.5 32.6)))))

